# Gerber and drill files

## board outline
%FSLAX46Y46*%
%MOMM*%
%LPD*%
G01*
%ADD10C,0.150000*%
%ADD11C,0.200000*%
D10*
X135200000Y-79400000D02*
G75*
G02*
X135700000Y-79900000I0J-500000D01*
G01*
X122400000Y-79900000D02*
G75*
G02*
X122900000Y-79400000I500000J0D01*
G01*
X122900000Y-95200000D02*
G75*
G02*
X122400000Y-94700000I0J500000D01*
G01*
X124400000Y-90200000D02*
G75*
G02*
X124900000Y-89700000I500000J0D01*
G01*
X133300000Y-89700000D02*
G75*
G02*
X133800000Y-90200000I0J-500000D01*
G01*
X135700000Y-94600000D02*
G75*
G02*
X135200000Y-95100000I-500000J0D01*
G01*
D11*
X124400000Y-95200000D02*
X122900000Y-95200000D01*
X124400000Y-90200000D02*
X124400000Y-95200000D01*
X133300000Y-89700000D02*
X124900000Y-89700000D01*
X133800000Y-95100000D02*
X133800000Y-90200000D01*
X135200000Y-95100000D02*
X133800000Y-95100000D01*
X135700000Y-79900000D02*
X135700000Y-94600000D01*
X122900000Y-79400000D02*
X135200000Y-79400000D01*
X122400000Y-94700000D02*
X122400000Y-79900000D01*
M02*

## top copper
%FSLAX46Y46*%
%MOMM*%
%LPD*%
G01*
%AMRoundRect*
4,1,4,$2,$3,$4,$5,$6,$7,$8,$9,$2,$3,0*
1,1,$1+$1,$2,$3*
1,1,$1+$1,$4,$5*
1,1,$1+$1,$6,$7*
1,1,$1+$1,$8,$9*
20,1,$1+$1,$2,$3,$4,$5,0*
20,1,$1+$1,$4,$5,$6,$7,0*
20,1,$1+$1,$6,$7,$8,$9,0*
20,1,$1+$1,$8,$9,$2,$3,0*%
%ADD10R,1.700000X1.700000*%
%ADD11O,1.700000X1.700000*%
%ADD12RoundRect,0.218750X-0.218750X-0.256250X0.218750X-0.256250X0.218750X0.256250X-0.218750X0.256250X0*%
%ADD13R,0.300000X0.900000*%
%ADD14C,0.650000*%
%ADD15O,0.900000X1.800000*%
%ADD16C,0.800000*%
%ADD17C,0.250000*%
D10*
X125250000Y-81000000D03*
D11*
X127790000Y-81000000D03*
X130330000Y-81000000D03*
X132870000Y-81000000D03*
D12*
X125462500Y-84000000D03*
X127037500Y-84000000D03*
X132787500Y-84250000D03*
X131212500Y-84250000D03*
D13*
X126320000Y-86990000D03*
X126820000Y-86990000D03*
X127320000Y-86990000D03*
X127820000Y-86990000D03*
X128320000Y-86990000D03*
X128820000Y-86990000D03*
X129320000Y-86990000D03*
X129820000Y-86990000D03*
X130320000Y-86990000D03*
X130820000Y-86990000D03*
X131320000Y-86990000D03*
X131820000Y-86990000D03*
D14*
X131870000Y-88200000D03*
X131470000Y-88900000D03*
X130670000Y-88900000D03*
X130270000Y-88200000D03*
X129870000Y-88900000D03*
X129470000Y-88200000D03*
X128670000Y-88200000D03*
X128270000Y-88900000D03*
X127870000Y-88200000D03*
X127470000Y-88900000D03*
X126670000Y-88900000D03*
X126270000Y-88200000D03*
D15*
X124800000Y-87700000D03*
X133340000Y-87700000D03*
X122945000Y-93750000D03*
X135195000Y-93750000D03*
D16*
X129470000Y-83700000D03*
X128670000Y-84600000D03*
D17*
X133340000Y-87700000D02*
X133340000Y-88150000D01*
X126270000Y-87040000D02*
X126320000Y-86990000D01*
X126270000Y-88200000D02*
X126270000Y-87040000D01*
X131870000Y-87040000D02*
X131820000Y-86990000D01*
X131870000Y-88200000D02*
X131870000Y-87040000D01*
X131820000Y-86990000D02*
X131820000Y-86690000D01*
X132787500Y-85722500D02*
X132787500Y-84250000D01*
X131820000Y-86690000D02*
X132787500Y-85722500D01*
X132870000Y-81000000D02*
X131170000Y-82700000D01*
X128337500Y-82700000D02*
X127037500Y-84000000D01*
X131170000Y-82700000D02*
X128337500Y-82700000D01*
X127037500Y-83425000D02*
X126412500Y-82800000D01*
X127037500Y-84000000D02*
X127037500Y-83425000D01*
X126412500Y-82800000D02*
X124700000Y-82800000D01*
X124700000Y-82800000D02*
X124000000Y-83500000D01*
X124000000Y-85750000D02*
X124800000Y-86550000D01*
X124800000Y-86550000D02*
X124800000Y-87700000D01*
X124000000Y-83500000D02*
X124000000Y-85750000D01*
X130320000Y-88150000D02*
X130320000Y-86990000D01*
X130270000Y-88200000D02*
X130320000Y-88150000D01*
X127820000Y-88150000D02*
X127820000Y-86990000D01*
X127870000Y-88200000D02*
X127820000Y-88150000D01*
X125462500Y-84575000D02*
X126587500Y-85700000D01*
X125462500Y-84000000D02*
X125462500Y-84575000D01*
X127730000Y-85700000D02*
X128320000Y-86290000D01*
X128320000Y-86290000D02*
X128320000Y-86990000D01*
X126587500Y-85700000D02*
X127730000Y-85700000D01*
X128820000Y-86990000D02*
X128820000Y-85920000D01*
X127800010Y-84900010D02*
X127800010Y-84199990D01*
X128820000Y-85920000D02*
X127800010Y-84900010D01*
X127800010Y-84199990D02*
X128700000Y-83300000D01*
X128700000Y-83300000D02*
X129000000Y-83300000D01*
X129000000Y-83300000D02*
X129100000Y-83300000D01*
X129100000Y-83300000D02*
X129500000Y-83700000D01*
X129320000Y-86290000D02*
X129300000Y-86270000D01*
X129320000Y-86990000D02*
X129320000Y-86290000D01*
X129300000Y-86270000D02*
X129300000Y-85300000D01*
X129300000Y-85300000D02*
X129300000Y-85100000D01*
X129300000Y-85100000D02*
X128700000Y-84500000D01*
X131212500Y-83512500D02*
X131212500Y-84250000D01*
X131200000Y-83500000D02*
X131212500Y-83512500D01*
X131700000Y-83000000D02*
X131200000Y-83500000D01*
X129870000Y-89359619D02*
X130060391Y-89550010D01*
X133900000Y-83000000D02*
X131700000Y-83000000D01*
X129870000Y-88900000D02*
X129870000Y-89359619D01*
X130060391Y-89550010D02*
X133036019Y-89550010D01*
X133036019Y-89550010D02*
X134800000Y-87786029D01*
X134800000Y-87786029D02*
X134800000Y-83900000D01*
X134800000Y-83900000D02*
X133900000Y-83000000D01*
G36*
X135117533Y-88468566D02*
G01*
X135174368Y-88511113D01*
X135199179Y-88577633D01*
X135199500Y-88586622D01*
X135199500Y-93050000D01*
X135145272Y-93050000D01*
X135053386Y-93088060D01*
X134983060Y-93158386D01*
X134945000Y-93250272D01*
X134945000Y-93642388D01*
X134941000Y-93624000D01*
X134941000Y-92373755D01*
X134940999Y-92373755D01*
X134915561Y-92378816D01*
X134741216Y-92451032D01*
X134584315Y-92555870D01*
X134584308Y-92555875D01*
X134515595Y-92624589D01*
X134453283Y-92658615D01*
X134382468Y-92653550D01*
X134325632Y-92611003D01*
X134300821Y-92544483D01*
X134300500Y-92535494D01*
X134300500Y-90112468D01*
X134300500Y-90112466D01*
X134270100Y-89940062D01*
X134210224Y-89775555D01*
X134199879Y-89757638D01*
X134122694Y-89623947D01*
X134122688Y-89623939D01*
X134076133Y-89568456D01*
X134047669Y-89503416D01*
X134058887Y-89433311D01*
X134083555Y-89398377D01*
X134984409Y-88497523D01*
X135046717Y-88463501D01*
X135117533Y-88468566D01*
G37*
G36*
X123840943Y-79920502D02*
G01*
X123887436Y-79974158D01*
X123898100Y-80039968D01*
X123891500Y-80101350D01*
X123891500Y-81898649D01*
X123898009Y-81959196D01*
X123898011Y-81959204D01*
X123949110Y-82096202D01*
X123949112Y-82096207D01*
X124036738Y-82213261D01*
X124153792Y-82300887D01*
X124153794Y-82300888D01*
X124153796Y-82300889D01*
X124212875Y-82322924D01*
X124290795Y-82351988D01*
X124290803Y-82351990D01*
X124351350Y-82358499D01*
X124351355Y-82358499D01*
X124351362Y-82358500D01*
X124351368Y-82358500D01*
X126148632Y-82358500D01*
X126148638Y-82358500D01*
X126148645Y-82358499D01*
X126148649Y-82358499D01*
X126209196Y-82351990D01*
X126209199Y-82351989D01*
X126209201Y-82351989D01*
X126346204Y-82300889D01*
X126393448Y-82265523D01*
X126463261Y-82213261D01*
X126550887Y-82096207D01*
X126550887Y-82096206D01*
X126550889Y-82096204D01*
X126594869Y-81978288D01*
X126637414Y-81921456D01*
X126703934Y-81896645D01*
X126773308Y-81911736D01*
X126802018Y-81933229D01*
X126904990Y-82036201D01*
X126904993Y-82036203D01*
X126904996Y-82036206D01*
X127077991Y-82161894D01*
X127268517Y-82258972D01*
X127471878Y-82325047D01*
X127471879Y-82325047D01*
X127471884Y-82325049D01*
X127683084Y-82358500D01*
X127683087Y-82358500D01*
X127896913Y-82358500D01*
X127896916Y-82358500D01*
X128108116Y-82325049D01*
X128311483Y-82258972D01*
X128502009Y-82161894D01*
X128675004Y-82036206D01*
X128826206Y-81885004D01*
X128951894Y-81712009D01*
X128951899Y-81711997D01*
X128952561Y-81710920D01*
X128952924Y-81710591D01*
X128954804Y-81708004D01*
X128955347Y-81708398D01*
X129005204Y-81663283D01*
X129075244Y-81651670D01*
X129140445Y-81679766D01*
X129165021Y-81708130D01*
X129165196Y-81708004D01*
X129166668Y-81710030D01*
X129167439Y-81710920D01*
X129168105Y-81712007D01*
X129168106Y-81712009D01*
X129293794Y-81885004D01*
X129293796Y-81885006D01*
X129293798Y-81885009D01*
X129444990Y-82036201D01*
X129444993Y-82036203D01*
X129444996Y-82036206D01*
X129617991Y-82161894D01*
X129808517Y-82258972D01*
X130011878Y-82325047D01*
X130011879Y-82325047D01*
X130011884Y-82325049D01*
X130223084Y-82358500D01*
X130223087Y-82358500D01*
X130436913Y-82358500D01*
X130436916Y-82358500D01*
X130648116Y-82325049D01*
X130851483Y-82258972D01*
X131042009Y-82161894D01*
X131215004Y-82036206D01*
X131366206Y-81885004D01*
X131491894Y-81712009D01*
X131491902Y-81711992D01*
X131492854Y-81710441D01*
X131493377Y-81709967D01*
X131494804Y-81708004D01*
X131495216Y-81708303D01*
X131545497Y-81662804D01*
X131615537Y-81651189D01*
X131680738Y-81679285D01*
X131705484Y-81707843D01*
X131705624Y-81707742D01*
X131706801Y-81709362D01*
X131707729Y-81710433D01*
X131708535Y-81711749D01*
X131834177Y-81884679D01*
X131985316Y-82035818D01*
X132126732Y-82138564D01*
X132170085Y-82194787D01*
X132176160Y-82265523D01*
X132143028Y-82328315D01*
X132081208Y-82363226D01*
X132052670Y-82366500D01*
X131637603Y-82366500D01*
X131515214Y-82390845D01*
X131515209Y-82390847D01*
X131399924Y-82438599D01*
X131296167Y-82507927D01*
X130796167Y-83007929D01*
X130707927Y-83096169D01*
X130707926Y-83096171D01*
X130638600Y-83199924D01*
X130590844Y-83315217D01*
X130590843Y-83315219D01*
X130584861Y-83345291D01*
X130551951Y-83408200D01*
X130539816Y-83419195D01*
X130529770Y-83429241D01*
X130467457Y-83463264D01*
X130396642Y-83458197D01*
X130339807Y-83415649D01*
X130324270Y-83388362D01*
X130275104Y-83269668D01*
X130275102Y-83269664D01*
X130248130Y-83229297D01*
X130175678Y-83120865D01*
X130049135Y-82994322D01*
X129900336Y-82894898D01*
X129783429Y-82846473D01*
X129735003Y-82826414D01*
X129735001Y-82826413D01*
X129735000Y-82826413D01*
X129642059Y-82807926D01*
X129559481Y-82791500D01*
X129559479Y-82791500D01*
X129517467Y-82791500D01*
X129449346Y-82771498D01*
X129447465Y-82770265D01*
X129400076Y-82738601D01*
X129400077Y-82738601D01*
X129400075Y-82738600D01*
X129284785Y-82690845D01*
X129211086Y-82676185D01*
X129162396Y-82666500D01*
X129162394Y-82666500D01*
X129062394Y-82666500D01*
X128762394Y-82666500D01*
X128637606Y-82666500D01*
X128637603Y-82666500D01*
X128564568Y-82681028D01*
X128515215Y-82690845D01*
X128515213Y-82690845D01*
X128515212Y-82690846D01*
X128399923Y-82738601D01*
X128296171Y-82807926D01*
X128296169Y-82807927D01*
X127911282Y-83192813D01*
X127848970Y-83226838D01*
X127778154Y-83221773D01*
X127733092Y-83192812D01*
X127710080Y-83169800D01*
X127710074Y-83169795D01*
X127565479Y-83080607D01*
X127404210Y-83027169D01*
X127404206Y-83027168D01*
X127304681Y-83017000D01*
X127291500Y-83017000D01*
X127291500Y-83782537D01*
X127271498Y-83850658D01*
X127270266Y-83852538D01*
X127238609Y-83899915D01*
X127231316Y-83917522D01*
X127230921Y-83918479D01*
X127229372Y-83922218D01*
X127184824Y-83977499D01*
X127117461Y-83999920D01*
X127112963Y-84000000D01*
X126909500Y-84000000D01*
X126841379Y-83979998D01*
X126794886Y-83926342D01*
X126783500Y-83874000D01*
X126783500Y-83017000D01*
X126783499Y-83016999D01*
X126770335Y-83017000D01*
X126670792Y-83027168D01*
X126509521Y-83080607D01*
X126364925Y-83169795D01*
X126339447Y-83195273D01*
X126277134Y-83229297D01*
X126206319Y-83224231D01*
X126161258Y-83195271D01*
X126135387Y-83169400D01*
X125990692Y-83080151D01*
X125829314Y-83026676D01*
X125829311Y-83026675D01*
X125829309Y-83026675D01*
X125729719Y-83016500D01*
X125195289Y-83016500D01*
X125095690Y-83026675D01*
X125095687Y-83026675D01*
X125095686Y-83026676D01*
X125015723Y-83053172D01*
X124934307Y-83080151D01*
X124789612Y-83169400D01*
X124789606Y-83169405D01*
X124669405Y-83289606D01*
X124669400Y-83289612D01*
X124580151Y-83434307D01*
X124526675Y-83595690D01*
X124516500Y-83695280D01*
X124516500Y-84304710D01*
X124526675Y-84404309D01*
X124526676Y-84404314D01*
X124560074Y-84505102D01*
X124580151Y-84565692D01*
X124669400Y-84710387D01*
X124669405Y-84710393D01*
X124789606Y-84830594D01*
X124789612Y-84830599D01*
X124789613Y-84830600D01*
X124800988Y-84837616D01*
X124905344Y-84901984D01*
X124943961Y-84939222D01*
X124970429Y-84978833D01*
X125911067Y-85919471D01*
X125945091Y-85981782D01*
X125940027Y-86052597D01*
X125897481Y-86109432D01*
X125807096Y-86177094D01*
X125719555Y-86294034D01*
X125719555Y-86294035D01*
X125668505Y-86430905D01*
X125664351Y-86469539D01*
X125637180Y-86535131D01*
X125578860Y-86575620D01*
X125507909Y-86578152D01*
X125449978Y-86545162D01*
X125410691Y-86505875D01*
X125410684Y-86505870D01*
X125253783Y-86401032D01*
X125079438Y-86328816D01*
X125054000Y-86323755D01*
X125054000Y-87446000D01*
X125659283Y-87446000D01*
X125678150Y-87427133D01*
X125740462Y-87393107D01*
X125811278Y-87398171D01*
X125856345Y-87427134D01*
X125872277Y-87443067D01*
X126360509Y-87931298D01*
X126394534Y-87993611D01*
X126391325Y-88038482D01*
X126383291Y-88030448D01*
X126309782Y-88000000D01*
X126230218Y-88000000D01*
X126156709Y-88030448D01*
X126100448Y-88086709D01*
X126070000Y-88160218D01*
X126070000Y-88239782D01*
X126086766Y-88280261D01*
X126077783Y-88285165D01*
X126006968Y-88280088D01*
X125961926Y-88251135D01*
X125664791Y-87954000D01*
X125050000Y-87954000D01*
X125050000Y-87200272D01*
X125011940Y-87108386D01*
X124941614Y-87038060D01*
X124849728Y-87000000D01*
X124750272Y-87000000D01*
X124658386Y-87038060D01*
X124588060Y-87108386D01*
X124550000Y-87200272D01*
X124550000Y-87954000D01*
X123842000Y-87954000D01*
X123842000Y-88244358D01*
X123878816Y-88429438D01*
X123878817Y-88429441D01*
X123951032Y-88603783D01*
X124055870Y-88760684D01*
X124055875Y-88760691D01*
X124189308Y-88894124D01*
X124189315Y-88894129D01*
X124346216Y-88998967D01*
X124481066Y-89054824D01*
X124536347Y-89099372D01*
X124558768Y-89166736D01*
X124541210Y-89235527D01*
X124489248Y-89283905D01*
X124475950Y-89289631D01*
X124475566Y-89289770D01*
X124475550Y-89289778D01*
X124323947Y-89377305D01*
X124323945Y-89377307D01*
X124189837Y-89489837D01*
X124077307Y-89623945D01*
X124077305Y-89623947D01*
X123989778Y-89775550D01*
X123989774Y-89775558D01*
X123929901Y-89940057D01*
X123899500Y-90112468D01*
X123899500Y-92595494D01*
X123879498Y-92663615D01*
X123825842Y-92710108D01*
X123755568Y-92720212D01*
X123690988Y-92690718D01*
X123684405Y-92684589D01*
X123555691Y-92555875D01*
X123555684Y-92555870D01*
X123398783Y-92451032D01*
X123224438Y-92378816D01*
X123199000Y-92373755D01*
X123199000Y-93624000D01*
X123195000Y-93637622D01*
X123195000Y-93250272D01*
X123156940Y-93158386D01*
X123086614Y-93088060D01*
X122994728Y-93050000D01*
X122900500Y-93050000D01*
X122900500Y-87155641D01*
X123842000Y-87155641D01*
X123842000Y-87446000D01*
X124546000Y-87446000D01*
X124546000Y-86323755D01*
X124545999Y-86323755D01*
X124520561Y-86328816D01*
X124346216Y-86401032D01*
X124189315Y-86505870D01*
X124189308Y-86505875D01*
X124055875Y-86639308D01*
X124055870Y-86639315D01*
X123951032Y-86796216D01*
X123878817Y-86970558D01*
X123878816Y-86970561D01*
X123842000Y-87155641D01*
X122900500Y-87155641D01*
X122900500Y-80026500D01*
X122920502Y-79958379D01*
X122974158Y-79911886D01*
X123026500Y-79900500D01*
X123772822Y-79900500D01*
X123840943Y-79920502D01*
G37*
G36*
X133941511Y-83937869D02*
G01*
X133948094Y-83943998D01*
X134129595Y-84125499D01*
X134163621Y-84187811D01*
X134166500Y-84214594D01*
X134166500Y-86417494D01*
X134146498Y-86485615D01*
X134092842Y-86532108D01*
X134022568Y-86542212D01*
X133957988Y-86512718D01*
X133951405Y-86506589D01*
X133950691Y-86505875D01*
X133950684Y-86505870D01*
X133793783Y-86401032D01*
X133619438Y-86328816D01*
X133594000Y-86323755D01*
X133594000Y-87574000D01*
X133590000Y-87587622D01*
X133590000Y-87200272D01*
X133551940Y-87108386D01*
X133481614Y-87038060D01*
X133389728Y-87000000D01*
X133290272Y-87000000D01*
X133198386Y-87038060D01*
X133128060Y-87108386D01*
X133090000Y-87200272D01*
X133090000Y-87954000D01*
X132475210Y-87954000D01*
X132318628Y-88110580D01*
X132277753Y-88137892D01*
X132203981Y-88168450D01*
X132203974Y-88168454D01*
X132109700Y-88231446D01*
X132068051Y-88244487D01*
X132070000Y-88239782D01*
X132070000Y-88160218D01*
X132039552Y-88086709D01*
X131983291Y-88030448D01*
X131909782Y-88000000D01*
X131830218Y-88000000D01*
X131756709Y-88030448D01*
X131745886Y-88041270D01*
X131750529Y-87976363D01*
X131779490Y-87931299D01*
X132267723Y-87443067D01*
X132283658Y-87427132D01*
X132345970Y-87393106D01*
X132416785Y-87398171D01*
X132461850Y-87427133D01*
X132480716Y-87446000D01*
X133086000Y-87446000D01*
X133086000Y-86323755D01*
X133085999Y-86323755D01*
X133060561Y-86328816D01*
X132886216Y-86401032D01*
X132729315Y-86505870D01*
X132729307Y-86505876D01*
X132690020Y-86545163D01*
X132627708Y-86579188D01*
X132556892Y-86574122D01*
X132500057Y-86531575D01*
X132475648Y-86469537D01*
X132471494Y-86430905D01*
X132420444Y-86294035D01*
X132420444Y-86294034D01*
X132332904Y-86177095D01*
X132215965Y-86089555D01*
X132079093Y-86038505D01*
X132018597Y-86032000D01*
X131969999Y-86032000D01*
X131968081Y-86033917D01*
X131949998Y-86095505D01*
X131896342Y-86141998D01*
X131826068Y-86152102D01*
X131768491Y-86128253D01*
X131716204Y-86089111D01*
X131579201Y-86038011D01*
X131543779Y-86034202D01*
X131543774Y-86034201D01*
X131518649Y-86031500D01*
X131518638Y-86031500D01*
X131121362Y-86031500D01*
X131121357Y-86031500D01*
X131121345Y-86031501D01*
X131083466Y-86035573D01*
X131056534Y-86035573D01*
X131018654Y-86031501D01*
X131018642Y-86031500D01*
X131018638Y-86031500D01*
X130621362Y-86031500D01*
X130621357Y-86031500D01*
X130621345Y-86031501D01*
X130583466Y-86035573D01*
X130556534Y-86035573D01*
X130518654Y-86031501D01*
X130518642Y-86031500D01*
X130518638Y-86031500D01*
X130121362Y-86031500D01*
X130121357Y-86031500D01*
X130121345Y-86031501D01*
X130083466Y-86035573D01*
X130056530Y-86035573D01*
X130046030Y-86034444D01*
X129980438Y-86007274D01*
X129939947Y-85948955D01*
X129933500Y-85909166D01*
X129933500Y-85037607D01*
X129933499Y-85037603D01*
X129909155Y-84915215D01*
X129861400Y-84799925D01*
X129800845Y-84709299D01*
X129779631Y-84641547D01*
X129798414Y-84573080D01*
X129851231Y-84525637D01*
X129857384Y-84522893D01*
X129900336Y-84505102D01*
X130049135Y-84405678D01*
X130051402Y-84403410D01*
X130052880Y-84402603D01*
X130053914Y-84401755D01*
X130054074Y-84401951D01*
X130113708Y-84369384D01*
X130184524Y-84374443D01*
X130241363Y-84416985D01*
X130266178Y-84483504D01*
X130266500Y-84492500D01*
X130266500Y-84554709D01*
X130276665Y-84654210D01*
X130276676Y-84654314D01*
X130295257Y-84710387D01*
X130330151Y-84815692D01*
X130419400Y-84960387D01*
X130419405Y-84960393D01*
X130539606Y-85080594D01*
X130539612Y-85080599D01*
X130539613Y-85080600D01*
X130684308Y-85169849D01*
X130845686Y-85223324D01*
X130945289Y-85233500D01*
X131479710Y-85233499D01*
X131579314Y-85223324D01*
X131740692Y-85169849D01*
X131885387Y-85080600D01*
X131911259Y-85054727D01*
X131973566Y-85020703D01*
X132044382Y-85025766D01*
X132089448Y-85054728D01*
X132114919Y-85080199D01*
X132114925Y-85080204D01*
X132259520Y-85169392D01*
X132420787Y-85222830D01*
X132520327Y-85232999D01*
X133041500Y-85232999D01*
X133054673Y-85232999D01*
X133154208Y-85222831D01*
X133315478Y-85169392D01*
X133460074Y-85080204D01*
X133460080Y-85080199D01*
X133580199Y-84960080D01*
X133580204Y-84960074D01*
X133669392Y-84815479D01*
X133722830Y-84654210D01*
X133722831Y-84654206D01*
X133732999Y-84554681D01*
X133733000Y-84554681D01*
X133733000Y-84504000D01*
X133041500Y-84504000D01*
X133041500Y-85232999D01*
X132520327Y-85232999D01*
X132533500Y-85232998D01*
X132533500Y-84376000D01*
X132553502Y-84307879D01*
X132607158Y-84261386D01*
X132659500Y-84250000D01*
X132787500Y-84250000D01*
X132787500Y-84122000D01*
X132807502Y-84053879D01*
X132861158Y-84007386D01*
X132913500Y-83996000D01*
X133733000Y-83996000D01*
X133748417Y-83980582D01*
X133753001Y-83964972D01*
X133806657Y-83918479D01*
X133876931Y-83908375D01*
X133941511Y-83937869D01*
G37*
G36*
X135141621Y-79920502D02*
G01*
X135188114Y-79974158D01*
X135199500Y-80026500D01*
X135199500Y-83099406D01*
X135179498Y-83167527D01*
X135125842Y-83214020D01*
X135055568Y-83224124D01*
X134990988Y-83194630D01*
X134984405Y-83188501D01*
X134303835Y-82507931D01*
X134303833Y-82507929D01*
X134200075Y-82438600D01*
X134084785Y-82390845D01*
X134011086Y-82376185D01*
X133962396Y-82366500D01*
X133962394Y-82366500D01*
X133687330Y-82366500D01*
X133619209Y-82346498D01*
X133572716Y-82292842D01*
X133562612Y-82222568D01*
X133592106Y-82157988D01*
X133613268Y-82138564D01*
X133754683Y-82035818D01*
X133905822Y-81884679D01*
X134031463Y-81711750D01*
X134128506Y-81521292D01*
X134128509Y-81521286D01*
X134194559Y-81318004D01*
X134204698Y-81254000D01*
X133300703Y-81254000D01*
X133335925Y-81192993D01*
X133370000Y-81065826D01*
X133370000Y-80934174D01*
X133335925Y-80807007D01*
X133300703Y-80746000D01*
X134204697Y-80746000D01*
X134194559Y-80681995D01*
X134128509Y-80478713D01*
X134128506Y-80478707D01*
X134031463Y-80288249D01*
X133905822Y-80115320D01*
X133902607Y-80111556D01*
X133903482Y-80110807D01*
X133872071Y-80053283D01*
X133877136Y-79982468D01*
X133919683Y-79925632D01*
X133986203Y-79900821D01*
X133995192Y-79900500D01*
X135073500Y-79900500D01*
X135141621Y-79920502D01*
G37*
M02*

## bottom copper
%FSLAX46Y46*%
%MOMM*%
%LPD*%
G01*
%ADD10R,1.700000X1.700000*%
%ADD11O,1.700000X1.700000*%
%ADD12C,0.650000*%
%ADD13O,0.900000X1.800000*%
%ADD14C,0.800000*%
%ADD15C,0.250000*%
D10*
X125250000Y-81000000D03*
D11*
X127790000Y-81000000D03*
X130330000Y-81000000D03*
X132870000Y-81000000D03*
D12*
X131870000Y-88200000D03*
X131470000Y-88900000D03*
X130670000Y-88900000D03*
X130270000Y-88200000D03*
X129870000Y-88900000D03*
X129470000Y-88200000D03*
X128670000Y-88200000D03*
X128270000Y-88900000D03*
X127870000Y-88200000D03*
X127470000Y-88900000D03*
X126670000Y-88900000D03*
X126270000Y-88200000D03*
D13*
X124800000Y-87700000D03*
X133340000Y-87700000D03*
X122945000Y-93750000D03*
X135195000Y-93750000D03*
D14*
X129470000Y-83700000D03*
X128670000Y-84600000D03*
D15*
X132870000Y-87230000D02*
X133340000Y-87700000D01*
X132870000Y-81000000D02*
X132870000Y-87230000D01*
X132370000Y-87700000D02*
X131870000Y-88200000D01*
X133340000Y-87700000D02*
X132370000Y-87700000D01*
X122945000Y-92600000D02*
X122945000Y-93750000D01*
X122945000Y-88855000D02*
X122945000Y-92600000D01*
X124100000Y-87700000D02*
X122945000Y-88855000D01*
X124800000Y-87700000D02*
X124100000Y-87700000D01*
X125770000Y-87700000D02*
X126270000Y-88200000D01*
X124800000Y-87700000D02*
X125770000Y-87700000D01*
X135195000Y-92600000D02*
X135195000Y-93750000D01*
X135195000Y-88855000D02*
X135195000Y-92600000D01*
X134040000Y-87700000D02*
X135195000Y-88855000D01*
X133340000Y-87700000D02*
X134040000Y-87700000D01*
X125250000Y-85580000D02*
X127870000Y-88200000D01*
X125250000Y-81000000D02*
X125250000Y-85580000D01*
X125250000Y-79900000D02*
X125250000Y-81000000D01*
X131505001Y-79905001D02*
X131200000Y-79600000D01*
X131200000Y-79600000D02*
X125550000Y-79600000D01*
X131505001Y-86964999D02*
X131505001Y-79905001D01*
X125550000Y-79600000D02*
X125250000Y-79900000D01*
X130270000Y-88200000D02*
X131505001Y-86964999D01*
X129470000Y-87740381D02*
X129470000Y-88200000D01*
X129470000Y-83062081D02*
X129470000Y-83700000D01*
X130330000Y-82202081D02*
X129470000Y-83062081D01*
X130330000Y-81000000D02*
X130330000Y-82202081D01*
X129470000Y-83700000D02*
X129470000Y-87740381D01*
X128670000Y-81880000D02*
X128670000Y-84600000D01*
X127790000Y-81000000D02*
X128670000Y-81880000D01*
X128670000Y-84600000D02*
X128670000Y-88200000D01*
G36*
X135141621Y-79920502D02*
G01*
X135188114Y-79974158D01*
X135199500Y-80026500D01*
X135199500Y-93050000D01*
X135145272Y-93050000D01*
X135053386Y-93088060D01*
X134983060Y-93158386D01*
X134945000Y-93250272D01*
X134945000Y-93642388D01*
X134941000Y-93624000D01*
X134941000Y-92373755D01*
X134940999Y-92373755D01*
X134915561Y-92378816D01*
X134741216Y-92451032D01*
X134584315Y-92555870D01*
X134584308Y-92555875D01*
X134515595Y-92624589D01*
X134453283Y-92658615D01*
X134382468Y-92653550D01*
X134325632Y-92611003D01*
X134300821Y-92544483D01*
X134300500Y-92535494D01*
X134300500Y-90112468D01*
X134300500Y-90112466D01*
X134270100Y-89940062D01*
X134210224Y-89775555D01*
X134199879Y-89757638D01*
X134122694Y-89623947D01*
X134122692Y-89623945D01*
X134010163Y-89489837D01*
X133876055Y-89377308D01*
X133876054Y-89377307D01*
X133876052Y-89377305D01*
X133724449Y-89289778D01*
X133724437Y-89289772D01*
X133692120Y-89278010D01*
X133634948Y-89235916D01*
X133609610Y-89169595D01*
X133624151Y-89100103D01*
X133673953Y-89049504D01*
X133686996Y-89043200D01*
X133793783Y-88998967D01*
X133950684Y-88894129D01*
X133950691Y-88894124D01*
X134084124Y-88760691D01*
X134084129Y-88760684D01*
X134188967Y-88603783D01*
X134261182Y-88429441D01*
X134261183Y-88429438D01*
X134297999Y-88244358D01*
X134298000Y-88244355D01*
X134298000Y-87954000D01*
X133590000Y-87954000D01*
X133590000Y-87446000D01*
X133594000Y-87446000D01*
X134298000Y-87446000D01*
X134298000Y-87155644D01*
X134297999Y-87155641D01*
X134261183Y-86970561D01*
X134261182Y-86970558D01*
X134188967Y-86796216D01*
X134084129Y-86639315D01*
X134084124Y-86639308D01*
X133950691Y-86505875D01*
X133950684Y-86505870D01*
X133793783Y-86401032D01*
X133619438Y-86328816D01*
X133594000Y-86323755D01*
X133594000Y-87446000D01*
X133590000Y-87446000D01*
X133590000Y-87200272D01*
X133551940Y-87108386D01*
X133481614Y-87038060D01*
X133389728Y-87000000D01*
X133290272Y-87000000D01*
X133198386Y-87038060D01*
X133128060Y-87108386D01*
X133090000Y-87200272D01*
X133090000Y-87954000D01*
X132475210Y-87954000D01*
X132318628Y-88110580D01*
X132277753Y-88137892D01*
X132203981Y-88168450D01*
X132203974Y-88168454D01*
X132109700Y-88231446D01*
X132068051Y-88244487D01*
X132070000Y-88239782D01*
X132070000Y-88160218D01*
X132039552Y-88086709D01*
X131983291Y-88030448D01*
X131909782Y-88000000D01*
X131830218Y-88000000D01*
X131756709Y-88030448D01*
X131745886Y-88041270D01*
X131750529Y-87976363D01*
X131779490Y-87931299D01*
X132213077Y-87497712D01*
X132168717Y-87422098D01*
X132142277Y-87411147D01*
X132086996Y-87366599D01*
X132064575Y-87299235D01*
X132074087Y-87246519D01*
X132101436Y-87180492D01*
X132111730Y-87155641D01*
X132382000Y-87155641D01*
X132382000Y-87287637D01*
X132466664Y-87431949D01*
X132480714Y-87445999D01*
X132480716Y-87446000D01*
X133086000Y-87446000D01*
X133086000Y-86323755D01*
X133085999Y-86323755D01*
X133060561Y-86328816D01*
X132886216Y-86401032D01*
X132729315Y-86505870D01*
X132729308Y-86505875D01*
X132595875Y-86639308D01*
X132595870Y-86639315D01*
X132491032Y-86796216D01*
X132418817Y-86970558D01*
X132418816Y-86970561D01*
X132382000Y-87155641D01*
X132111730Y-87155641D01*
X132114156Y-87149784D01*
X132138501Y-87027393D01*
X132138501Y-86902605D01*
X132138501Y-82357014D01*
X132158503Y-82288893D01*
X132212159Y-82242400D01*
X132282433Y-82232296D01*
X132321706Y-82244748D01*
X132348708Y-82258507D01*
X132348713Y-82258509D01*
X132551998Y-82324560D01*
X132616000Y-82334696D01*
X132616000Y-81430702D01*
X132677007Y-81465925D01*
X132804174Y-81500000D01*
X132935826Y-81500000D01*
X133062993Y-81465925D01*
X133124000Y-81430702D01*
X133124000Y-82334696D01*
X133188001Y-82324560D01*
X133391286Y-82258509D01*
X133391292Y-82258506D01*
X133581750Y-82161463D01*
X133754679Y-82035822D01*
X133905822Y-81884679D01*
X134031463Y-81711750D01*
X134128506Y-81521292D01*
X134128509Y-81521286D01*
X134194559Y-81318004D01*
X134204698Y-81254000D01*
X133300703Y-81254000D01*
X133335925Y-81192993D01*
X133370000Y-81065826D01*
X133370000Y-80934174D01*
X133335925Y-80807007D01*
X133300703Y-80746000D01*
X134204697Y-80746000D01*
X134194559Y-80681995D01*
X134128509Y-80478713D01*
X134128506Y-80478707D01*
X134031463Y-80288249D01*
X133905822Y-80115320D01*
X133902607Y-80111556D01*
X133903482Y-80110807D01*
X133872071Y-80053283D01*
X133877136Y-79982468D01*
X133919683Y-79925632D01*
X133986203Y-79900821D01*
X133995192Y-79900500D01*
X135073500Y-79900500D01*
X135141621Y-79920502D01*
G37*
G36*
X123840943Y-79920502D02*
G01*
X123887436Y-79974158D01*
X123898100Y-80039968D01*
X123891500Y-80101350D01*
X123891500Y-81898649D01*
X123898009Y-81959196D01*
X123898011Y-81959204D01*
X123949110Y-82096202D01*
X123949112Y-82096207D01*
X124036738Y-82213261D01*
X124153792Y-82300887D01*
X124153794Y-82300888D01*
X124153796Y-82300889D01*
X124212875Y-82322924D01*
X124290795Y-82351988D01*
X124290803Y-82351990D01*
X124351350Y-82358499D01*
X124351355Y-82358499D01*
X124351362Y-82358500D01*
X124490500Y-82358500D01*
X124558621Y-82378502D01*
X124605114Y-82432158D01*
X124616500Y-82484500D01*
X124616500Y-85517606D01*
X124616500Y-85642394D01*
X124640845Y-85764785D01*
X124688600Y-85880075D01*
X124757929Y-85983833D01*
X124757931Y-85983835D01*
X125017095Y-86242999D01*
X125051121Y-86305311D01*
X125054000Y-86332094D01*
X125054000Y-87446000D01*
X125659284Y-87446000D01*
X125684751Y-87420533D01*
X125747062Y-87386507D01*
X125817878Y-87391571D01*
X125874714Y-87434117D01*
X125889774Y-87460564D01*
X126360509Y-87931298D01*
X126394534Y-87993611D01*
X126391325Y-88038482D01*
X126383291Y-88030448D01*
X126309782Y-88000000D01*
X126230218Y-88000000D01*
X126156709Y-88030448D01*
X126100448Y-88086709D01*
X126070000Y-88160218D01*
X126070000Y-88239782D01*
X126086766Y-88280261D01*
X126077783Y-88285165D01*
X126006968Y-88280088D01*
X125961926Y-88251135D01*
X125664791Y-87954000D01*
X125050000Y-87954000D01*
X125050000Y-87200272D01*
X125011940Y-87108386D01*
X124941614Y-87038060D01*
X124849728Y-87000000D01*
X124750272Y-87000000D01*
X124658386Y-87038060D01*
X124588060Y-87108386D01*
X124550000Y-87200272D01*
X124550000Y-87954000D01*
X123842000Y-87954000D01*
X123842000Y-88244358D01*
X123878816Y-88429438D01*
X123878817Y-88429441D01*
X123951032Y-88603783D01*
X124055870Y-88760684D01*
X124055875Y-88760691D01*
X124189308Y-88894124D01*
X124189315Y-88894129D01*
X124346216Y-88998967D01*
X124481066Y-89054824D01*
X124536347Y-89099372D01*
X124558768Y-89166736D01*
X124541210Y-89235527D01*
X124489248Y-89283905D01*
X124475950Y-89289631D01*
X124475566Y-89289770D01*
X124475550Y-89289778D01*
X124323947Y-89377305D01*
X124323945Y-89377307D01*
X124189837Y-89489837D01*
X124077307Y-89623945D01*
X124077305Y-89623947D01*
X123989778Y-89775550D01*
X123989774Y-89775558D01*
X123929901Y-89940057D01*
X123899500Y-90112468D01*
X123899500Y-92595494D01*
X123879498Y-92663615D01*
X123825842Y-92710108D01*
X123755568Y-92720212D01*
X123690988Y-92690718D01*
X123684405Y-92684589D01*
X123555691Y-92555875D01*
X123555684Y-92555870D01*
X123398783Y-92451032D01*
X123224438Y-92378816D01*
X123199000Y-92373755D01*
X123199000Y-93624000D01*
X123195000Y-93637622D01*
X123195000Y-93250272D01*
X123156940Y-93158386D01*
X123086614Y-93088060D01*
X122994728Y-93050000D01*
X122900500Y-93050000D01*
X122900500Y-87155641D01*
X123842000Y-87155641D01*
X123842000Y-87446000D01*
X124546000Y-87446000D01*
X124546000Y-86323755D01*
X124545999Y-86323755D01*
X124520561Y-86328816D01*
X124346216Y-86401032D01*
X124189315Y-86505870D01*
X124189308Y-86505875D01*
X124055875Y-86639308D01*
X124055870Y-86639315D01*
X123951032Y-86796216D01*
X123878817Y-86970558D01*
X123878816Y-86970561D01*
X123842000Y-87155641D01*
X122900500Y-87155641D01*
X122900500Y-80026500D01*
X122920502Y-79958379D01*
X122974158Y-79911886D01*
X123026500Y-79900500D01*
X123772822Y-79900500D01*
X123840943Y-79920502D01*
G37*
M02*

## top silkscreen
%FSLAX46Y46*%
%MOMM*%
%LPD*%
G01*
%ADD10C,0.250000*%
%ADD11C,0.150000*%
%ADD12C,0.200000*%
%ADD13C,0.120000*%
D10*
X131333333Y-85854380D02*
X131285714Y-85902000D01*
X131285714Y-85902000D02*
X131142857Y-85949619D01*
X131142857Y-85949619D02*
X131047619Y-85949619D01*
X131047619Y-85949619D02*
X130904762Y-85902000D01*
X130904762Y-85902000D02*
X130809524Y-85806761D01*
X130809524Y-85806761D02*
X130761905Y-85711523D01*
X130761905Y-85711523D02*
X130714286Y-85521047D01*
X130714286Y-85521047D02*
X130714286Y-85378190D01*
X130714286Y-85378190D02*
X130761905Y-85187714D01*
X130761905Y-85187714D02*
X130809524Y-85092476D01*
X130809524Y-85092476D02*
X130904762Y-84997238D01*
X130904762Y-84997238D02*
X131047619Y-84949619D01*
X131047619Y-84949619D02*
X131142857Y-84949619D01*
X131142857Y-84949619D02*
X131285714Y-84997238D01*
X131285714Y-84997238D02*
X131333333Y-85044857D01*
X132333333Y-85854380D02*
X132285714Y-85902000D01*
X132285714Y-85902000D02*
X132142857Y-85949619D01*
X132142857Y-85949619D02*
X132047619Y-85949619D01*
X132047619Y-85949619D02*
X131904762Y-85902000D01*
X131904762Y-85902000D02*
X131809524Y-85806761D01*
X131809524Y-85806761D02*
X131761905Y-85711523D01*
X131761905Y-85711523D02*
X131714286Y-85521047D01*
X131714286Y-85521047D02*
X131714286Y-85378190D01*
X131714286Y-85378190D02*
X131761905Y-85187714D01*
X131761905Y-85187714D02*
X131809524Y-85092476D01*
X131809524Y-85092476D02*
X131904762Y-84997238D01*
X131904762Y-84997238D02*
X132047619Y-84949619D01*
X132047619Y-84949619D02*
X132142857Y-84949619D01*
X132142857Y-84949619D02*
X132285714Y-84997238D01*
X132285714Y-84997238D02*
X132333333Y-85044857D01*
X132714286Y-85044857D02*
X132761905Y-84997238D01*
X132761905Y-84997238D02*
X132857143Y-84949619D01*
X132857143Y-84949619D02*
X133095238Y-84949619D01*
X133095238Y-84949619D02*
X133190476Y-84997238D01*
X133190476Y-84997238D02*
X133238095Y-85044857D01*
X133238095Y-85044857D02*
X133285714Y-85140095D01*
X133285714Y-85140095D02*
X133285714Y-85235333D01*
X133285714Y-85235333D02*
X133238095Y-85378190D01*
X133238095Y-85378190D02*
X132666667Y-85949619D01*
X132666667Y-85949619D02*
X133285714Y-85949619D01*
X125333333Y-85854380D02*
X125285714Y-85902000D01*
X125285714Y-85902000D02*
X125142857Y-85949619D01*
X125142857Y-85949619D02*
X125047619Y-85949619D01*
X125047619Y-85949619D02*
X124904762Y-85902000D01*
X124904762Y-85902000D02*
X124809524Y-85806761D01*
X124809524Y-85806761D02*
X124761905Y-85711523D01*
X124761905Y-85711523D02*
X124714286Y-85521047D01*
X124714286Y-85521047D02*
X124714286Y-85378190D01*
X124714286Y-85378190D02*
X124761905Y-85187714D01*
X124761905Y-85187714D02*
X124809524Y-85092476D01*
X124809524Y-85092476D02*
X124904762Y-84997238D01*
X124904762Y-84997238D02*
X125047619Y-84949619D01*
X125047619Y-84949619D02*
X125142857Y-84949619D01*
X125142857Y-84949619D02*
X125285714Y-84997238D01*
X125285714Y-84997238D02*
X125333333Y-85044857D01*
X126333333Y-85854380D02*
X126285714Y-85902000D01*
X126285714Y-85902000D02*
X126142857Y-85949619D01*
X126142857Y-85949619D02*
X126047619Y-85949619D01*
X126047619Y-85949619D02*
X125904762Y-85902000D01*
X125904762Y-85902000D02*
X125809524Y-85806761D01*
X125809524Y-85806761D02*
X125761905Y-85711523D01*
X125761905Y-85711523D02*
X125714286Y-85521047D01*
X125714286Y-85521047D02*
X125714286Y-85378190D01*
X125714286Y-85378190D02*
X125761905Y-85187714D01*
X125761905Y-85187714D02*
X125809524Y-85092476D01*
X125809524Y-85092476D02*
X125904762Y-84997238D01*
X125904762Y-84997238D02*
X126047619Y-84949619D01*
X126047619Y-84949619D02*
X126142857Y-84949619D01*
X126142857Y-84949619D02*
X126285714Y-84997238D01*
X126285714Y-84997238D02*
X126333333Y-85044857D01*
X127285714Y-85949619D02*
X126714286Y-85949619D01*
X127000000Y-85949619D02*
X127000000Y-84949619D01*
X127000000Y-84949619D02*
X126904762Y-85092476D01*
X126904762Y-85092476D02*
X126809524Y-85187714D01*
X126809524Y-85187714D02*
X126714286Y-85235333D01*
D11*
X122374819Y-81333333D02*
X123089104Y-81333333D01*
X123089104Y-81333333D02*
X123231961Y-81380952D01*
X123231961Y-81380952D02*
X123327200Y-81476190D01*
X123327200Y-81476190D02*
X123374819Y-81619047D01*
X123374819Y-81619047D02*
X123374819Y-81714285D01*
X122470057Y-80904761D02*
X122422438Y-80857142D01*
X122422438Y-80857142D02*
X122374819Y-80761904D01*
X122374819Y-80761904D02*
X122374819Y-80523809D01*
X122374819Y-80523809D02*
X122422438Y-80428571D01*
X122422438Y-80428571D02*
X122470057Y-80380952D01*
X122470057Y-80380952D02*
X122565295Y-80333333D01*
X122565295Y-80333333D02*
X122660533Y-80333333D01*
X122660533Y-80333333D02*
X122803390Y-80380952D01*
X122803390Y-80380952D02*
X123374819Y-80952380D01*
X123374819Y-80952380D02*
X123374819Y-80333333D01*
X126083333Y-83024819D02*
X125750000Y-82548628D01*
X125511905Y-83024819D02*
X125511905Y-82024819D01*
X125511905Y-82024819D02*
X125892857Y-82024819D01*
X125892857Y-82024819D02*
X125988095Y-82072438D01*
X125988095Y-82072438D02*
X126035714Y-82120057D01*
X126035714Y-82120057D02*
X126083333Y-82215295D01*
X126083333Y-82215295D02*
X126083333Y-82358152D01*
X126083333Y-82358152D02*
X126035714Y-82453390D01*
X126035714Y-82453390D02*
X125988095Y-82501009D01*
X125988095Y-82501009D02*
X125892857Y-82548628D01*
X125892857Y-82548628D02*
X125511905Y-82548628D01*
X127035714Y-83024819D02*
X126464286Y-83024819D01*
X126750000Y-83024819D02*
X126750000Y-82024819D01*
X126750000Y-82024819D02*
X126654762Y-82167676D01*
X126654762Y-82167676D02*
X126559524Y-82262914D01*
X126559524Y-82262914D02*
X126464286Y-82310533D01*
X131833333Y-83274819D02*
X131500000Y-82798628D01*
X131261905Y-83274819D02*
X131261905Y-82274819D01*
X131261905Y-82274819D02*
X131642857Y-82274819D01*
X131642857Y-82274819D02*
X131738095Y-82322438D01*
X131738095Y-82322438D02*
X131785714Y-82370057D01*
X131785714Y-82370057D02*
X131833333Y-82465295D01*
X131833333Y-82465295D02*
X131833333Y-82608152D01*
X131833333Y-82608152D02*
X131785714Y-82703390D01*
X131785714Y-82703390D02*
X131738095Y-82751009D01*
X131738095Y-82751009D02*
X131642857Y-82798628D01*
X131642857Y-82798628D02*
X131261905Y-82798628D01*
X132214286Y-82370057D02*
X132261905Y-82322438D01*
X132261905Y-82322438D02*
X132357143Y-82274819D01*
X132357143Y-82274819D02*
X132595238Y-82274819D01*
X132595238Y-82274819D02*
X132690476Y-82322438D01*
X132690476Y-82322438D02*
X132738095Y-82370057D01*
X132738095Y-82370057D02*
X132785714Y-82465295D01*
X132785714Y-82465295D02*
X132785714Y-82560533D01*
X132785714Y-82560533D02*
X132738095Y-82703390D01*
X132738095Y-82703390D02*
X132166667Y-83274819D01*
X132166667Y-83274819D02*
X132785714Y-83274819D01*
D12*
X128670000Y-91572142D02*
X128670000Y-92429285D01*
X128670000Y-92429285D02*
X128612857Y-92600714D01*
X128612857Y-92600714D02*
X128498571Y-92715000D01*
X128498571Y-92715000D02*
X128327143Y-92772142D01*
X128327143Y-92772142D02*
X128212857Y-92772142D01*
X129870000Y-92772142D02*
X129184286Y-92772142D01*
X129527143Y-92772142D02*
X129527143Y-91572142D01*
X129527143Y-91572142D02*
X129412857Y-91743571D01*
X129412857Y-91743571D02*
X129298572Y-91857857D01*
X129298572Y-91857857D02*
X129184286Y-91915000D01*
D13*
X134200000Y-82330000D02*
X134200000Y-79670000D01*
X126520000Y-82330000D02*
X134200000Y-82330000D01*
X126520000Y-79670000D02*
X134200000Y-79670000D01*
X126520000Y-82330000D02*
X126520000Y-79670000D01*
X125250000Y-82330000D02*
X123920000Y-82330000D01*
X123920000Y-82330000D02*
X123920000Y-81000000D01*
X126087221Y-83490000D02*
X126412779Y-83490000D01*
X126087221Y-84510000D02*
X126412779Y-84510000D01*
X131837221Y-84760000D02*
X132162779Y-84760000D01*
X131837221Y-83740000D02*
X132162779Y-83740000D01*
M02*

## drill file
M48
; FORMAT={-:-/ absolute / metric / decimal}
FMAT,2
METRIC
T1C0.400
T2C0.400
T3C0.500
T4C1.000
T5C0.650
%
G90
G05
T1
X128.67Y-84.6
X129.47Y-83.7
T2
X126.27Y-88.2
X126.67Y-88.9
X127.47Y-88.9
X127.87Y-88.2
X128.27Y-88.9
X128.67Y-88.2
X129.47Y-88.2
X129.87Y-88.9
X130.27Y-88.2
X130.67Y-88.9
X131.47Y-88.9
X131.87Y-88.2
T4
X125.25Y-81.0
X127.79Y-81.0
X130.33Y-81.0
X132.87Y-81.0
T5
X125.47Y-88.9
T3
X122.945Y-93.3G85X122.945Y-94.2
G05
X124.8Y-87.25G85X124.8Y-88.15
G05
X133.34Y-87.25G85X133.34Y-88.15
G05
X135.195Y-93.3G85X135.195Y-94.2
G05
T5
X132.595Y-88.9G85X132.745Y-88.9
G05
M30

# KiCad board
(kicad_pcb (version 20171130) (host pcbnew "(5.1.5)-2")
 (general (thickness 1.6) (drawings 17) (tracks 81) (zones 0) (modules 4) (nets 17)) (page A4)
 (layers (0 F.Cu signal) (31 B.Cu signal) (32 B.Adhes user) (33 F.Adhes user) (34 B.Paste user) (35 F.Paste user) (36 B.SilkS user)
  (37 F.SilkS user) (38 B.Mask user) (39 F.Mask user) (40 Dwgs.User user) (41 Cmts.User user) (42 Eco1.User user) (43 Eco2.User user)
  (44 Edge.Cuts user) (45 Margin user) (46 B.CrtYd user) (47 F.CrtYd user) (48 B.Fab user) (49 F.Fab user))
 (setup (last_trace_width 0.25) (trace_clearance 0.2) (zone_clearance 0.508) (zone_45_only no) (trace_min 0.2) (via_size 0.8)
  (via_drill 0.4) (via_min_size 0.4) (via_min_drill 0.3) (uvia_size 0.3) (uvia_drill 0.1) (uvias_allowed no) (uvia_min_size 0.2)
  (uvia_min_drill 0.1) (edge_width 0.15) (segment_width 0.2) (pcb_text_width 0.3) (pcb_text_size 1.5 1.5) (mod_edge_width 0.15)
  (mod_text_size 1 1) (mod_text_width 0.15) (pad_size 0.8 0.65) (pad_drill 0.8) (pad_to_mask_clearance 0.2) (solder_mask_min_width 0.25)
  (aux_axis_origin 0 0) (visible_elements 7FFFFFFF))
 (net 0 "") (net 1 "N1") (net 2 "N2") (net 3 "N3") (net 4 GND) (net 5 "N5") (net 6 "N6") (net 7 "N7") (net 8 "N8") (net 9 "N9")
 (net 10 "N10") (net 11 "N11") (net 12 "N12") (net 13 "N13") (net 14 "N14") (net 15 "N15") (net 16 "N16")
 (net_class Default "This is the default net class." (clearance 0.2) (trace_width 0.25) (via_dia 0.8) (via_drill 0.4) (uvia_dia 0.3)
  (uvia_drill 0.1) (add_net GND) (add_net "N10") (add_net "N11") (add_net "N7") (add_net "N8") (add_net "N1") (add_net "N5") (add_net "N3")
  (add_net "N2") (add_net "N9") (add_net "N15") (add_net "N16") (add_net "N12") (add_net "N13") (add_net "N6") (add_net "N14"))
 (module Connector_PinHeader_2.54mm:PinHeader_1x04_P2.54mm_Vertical (layer F.Cu) (at 125.25 81 90)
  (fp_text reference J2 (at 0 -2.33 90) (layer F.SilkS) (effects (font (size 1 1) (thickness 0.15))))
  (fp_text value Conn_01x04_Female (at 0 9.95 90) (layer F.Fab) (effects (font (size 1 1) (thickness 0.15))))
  (fp_line (start -1.33 8.95) (end 1.33 8.95) (layer F.SilkS) (width 0.12))
  (fp_line (start -1.33 1.27) (end -1.33 8.95) (layer F.SilkS) (width 0.12))
  (fp_line (start 1.33 1.27) (end 1.33 8.95) (layer F.SilkS) (width 0.12))
  (fp_line (start -1.33 1.27) (end 1.33 1.27) (layer F.SilkS) (width 0.12))
  (fp_line (start -1.33 0) (end -1.33 -1.33) (layer F.SilkS) (width 0.12))
  (fp_line (start -1.33 -1.33) (end 0 -1.33) (layer F.SilkS) (width 0.12))
  (pad 1 thru_hole rect (at 0 0 90) (size 1.7 1.7) (drill 1) (layers *.Cu *.Mask) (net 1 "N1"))
  (pad 2 thru_hole oval (at 0 2.54 90) (size 1.7 1.7) (drill 1) (layers *.Cu *.Mask) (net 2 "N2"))
  (pad 3 thru_hole oval (at 0 5.08 90) (size 1.7 1.7) (drill 1) (layers *.Cu *.Mask) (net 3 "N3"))
  (pad 4 thru_hole oval (at 0 7.62 90) (size 1.7 1.7) (drill 1) (layers *.Cu *.Mask) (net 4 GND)))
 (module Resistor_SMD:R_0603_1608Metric (layer F.Cu) (at 126.25 84)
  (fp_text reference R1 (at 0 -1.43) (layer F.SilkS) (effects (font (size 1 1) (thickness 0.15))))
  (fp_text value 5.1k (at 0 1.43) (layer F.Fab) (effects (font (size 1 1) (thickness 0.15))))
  (fp_line (start -0.162779 -0.51) (end 0.162779 -0.51) (layer F.SilkS) (width 0.12))
  (fp_line (start -0.162779 0.51) (end 0.162779 0.51) (layer F.SilkS) (width 0.12))
  (pad 1 smd roundrect (at -0.7875 0) (size 0.875 0.95) (layers F.Cu F.Paste F.Mask) (roundrect_rratio 0.25) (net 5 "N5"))
  (pad 2 smd roundrect (at 0.7875 0) (size 0.875 0.95) (layers F.Cu F.Paste F.Mask) (roundrect_rratio 0.25) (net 4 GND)))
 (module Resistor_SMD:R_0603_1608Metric (layer F.Cu) (at 132 84.25)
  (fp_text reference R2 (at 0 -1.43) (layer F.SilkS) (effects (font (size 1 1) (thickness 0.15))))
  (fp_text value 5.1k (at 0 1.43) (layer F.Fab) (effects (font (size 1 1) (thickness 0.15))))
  (fp_line (start -0.162779 0.51) (end 0.162779 0.51) (layer F.SilkS) (width 0.12))
  (fp_line (start -0.162779 -0.51) (end 0.162779 -0.51) (layer F.SilkS) (width 0.12))
  (pad 2 smd roundrect (at 0.7875 0) (size 0.875 0.95) (layers F.Cu F.Paste F.Mask) (roundrect_rratio 0.25) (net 4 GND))
  (pad 1 smd roundrect (at -0.7875 0) (size 0.875 0.95) (layers F.Cu F.Paste F.Mask) (roundrect_rratio 0.25) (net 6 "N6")))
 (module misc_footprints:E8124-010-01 (layer F.Cu) (at 129.07 88.9)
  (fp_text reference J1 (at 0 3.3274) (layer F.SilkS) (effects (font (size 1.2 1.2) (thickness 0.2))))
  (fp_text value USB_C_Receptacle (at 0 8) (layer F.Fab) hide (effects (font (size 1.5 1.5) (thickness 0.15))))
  (pad "" np_thru_hole circle (at -3.6 0) (size 0.65 0.65) (drill 0.65) (layers *.Cu *.Mask))
  (pad A1 smd rect (at -2.75 -1.91) (size 0.3 0.9) (layers F.Cu F.Paste F.Mask) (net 4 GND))
  (pad A2 smd rect (at -2.25 -1.91) (size 0.3 0.9) (layers F.Cu F.Paste F.Mask) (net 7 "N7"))
  (pad A3 smd rect (at -1.75 -1.91) (size 0.3 0.9) (layers F.Cu F.Paste F.Mask) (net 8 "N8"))
  (pad A4 smd rect (at -1.25 -1.91) (size 0.3 0.9) (layers F.Cu F.Paste F.Mask) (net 1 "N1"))
  (pad A5 smd rect (at -0.75 -1.91) (size 0.3 0.9) (layers F.Cu F.Paste F.Mask) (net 5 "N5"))
  (pad A6 smd rect (at -0.25 -1.91) (size 0.3 0.9) (layers F.Cu F.Paste F.Mask) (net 3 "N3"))
  (pad A7 smd rect (at 0.25 -1.91) (size 0.3 0.9) (layers F.Cu F.Paste F.Mask) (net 2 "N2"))
  (pad A8 smd rect (at 0.75 -1.91) (size 0.3 0.9) (layers F.Cu F.Paste F.Mask) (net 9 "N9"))
  (pad A9 smd rect (at 1.25 -1.91) (size 0.3 0.9) (layers F.Cu F.Paste F.Mask) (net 1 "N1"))
  (pad A10 smd rect (at 1.75 -1.91) (size 0.3 0.9) (layers F.Cu F.Paste F.Mask) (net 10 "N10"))
  (pad A11 smd rect (at 2.25 -1.91) (size 0.3 0.9) (layers F.Cu F.Paste F.Mask) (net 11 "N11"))
  (pad A12 smd rect (at 2.75 -1.91) (size 0.3 0.9) (layers F.Cu F.Paste F.Mask) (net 4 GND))
  (pad B1 thru_hole circle (at 2.8 -0.7) (size 0.65 0.65) (drill 0.4) (layers *.Cu *.Mask) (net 4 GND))
  (pad B2 thru_hole circle (at 2.4 0) (size 0.65 0.65) (drill 0.4) (layers *.Cu) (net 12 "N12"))
  (pad B3 thru_hole circle (at 1.6 0) (size 0.65 0.65) (drill 0.4) (layers *.Cu) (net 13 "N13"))
  (pad B4 thru_hole circle (at 1.2 -0.7) (size 0.65 0.65) (drill 0.4) (layers *.Cu *.Mask) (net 1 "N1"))
  (pad B5 thru_hole circle (at 0.8 0) (size 0.65 0.65) (drill 0.4) (layers *.Cu *.Mask) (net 6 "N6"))
  (pad B6 thru_hole circle (at 0.4 -0.7) (size 0.65 0.65) (drill 0.4) (layers *.Cu *.Mask) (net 3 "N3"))
  (pad B7 thru_hole circle (at -0.4 -0.7) (size 0.65 0.65) (drill 0.4) (layers *.Cu *.Mask) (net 2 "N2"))
  (pad B8 thru_hole circle (at -0.8 0) (size 0.65 0.65) (drill 0.4) (layers *.Cu *.Mask) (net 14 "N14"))
  (pad B9 thru_hole circle (at -1.2 -0.7) (size 0.65 0.65) (drill 0.4) (layers *.Cu *.Mask) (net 1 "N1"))
  (pad B10 thru_hole circle (at -1.6 0) (size 0.65 0.65) (drill 0.4) (layers *.Cu *.Mask) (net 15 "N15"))
  (pad B11 thru_hole circle (at -2.4 0) (size 0.65 0.65) (drill 0.4) (layers *.Cu *.Mask) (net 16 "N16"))
  (pad B12 thru_hole circle (at -2.8 -0.7) (size 0.65 0.65) (drill 0.4) (layers *.Cu *.Mask) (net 4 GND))
  (pad S1 thru_hole oval (at -4.27 -1.2) (size 0.9 1.8) (drill oval 0.5 1.4) (layers *.Cu *.Mask) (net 4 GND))
  (pad S1 thru_hole oval (at 4.27 -1.2) (size 0.9 1.8) (drill oval 0.5 1.4) (layers *.Cu *.Mask) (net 4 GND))
  (pad S1 thru_hole oval (at -6.125 4.85) (size 0.9 1.8) (drill oval 0.5 1.4) (layers *.Cu *.Mask) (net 4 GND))
  (pad S1 thru_hole oval (at 6.125 4.85) (size 0.9 1.8) (drill oval 0.5 1.4) (layers *.Cu *.Mask) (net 4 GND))
  (pad "" np_thru_hole oval (at 3.6 0) (size 0.8 0.65) (drill oval 0.8 0.65) (layers *.Cu)))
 (gr_arc (start 135.2 79.9) (end 135.7 79.9) (angle -90) (layer Edge.Cuts) (width 0.15))
 (gr_arc (start 122.9 79.9) (end 122.9 79.4) (angle -90) (layer Edge.Cuts) (width 0.15))
 (gr_arc (start 122.9 94.7) (end 122.4 94.7) (angle -90) (layer Edge.Cuts) (width 0.15))
 (gr_arc (start 124.9 90.2) (end 124.9 89.7) (angle -90) (layer Edge.Cuts) (width 0.15))
 (gr_arc (start 133.3 90.2) (end 133.8 90.2) (angle -90) (layer Edge.Cuts) (width 0.15))
 (gr_arc (start 135.2 94.6) (end 135.2 95.1) (angle -90) (layer Edge.Cuts) (width 0.15))
 (gr_line (start 124.4 95.2) (end 122.9 95.2) (layer Edge.Cuts) (width 0.2))
 (gr_line (start 124.4 90.2) (end 124.4 95.2) (layer Edge.Cuts) (width 0.2))
 (gr_line (start 133.3 89.7) (end 124.9 89.7) (layer Edge.Cuts) (width 0.2))
 (gr_line (start 133.8 95.1) (end 133.8 90.2) (layer Edge.Cuts) (width 0.2))
 (gr_line (start 135.2 95.1) (end 133.8 95.1) (layer Edge.Cuts) (width 0.2))
 (gr_line (start 135.7 79.9) (end 135.7 94.6) (layer Edge.Cuts) (width 0.2))
 (gr_line (start 122.9 79.4) (end 135.2 79.4) (layer Edge.Cuts) (width 0.2))
 (gr_line (start 122.4 94.7) (end 122.4 79.9) (layer Edge.Cuts) (width 0.2))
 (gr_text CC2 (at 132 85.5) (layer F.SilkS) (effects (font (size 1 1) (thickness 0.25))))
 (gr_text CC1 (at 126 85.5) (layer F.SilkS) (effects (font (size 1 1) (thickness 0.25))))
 (segment (start 132.87 87.23) (end 133.34 87.7) (width 0.25) (layer B.Cu) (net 4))
 (segment (start 132.87 81) (end 132.87 87.23) (width 0.25) (layer B.Cu) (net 4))
 (segment (start 132.37 87.7) (end 131.87 88.2) (width 0.25) (layer B.Cu) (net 4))
 (segment (start 133.34 87.7) (end 132.37 87.7) (width 0.25) (layer B.Cu) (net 4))
 (segment (start 133.34 87.7) (end 133.34 88.15) (width 0.25) (layer F.Cu) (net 4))
 (segment (start 122.945 92.6) (end 122.945 93.75) (width 0.25) (layer B.Cu) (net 4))
 (segment (start 122.945 88.855) (end 122.945 92.6) (width 0.25) (layer B.Cu) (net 4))
 (segment (start 124.1 87.7) (end 122.945 88.855) (width 0.25) (layer B.Cu) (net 4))
 (segment (start 124.8 87.7) (end 124.1 87.7) (width 0.25) (layer B.Cu) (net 4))
 (segment (start 125.77 87.7) (end 126.27 88.2) (width 0.25) (layer B.Cu) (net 4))
 (segment (start 124.8 87.7) (end 125.77 87.7) (width 0.25) (layer B.Cu) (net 4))
 (segment (start 126.27 87.04) (end 126.32 86.99) (width 0.25) (layer F.Cu) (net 4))
 (segment (start 126.27 88.2) (end 126.27 87.04) (width 0.25) (layer F.Cu) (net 4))
 (segment (start 131.87 87.04) (end 131.82 86.99) (width 0.25) (layer F.Cu) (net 4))
 (segment (start 131.87 88.2) (end 131.87 87.04) (width 0.25) (layer F.Cu) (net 4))
 (segment (start 131.82 86.99) (end 131.82 86.69) (width 0.25) (layer F.Cu) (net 4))
 (segment (start 132.7875 85.7225) (end 132.7875 84.25) (width 0.25) (layer F.Cu) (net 4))
 (segment (start 131.82 86.69) (end 132.7875 85.7225) (width 0.25) (layer F.Cu) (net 4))
 (segment (start 132.87 81) (end 131.17 82.7) (width 0.25) (layer F.Cu) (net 4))
 (segment (start 128.3375 82.7) (end 127.0375 84) (width 0.25) (layer F.Cu) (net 4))
 (segment (start 131.17 82.7) (end 128.3375 82.7) (width 0.25) (layer F.Cu) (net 4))
 (segment (start 135.195 92.6) (end 135.195 93.75) (width 0.25) (layer B.Cu) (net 4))
 (segment (start 135.195 88.855) (end 135.195 92.6) (width 0.25) (layer B.Cu) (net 4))
 (segment (start 134.04 87.7) (end 135.195 88.855) (width 0.25) (layer B.Cu) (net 4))
 (segment (start 133.34 87.7) (end 134.04 87.7) (width 0.25) (layer B.Cu) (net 4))
 (segment (start 127.0375 83.425) (end 126.4125 82.8) (width 0.25) (layer F.Cu) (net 4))
 (segment (start 127.0375 84) (end 127.0375 83.425) (width 0.25) (layer F.Cu) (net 4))
 (segment (start 126.4125 82.8) (end 124.7 82.8) (width 0.25) (layer F.Cu) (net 4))
 (segment (start 124.7 82.8) (end 124 83.5) (width 0.25) (layer F.Cu) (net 4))
 (segment (start 124 85.75) (end 124.8 86.55) (width 0.25) (layer F.Cu) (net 4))
 (segment (start 124.8 86.55) (end 124.8 87.7) (width 0.25) (layer F.Cu) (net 4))
 (segment (start 124 83.5) (end 124 85.75) (width 0.25) (layer F.Cu) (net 4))
 (segment (start 125.25 85.58) (end 127.87 88.2) (width 0.25) (layer B.Cu) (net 1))
 (segment (start 125.25 81) (end 125.25 85.58) (width 0.25) (layer B.Cu) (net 1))
 (segment (start 130.32 88.15) (end 130.32 86.99) (width 0.25) (layer F.Cu) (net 1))
 (segment (start 130.27 88.2) (end 130.32 88.15) (width 0.25) (layer F.Cu) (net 1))
 (segment (start 127.82 88.15) (end 127.82 86.99) (width 0.25) (layer F.Cu) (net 1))
 (segment (start 127.87 88.2) (end 127.82 88.15) (width 0.25) (layer F.Cu) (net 1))
 (segment (start 125.25 79.9) (end 125.25 81) (width 0.25) (layer B.Cu) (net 1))
 (segment (start 131.505001 79.905001) (end 131.2 79.6) (width 0.25) (layer B.Cu) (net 1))
 (segment (start 131.2 79.6) (end 125.55 79.6) (width 0.25) (layer B.Cu) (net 1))
 (segment (start 131.505001 86.964999) (end 131.505001 79.905001) (width 0.25) (layer B.Cu) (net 1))
 (segment (start 125.55 79.6) (end 125.25 79.9) (width 0.25) (layer B.Cu) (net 1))
 (segment (start 130.27 88.2) (end 131.505001 86.964999) (width 0.25) (layer B.Cu) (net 1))
 (segment (start 125.4625 84.575) (end 126.5875 85.7) (width 0.25) (layer F.Cu) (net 5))
 (segment (start 125.4625 84) (end 125.4625 84.575) (width 0.25) (layer F.Cu) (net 5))
 (segment (start 127.73 85.7) (end 128.32 86.29) (width 0.25) (layer F.Cu) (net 5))
 (segment (start 128.32 86.29) (end 128.32 86.99) (width 0.25) (layer F.Cu) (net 5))
 (segment (start 126.5875 85.7) (end 127.73 85.7) (width 0.25) (layer F.Cu) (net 5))
 (segment (start 129.47 87.740381) (end 129.47 88.2) (width 0.25) (layer B.Cu) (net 3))
 (segment (start 129.47 83.062081) (end 129.47 83.7) (width 0.25) (layer B.Cu) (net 3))
 (segment (start 130.33 82.202081) (end 129.47 83.062081) (width 0.25) (layer B.Cu) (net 3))
 (segment (start 130.33 81) (end 130.33 82.202081) (width 0.25) (layer B.Cu) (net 3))
 (segment (start 128.82 86.99) (end 128.82 85.92) (width 0.25) (layer F.Cu) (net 3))
 (segment (start 127.80001 84.90001) (end 127.80001 84.19999) (width 0.25) (layer F.Cu) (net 3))
 (segment (start 128.82 85.92) (end 127.80001 84.90001) (width 0.25) (layer F.Cu) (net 3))
 (segment (start 127.80001 84.19999) (end 128.7 83.3) (width 0.25) (layer F.Cu) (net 3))
 (segment (start 128.7 83.3) (end 129 83.3) (width 0.25) (layer F.Cu) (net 3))
 (segment (start 129 83.3) (end 129.1 83.3) (width 0.25) (layer F.Cu) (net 3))
 (segment (start 129.1 83.3) (end 129.5 83.7) (width 0.25) (layer F.Cu) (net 3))
 (segment (start 129.47 83.7) (end 129.47 87.740381) (width 0.25) (layer B.Cu) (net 3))
 (via (at 129.47 83.7) (size 0.8) (drill 0.4) (layers F.Cu B.Cu) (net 3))
 (segment (start 128.67 81.88) (end 128.67 84.6) (width 0.25) (layer B.Cu) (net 2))
 (segment (start 127.79 81) (end 128.67 81.88) (width 0.25) (layer B.Cu) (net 2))
 (segment (start 129.32 86.29) (end 129.3 86.27) (width 0.25) (layer F.Cu) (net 2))
 (segment (start 129.32 86.99) (end 129.32 86.29) (width 0.25) (layer F.Cu) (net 2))
 (segment (start 129.3 86.27) (end 129.3 85.3) (width 0.25) (layer F.Cu) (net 2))
 (segment (start 129.3 85.3) (end 129.3 85.1) (width 0.25) (layer F.Cu) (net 2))
 (segment (start 129.3 85.1) (end 128.7 84.5) (width 0.25) (layer F.Cu) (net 2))
 (segment (start 128.67 84.6) (end 128.67 88.2) (width 0.25) (layer B.Cu) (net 2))
 (via (at 128.67 84.6) (size 0.8) (drill 0.4) (layers F.Cu B.Cu) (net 2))
 (segment (start 131.2125 83.5125) (end 131.2125 84.25) (width 0.25) (layer F.Cu) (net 6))
 (segment (start 131.2 83.5) (end 131.2125 83.5125) (width 0.25) (layer F.Cu) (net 6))
 (segment (start 131.7 83) (end 131.2 83.5) (width 0.25) (layer F.Cu) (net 6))
 (segment (start 129.87 89.359619) (end 130.060391 89.55001) (width 0.25) (layer F.Cu) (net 6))
 (segment (start 133.9 83) (end 131.7 83) (width 0.25) (layer F.Cu) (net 6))
 (segment (start 129.87 88.9) (end 129.87 89.359619) (width 0.25) (layer F.Cu) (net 6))
 (segment (start 130.060391 89.55001) (end 133.036019 89.55001) (width 0.25) (layer F.Cu) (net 6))
 (segment (start 133.036019 89.55001) (end 134.8 87.786029) (width 0.25) (layer F.Cu) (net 6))
 (segment (start 134.8 87.786029) (end 134.8 83.9) (width 0.25) (layer F.Cu) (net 6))
 (segment (start 134.8 83.9) (end 133.9 83) (width 0.25) (layer F.Cu) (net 6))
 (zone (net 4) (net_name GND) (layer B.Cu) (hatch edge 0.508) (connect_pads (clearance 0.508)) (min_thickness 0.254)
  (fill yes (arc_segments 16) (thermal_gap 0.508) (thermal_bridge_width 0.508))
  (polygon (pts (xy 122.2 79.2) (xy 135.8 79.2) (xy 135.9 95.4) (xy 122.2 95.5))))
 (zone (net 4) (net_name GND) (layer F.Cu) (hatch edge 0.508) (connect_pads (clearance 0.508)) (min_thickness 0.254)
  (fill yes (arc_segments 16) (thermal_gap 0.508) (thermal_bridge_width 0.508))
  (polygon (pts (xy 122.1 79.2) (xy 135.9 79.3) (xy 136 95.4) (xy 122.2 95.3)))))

